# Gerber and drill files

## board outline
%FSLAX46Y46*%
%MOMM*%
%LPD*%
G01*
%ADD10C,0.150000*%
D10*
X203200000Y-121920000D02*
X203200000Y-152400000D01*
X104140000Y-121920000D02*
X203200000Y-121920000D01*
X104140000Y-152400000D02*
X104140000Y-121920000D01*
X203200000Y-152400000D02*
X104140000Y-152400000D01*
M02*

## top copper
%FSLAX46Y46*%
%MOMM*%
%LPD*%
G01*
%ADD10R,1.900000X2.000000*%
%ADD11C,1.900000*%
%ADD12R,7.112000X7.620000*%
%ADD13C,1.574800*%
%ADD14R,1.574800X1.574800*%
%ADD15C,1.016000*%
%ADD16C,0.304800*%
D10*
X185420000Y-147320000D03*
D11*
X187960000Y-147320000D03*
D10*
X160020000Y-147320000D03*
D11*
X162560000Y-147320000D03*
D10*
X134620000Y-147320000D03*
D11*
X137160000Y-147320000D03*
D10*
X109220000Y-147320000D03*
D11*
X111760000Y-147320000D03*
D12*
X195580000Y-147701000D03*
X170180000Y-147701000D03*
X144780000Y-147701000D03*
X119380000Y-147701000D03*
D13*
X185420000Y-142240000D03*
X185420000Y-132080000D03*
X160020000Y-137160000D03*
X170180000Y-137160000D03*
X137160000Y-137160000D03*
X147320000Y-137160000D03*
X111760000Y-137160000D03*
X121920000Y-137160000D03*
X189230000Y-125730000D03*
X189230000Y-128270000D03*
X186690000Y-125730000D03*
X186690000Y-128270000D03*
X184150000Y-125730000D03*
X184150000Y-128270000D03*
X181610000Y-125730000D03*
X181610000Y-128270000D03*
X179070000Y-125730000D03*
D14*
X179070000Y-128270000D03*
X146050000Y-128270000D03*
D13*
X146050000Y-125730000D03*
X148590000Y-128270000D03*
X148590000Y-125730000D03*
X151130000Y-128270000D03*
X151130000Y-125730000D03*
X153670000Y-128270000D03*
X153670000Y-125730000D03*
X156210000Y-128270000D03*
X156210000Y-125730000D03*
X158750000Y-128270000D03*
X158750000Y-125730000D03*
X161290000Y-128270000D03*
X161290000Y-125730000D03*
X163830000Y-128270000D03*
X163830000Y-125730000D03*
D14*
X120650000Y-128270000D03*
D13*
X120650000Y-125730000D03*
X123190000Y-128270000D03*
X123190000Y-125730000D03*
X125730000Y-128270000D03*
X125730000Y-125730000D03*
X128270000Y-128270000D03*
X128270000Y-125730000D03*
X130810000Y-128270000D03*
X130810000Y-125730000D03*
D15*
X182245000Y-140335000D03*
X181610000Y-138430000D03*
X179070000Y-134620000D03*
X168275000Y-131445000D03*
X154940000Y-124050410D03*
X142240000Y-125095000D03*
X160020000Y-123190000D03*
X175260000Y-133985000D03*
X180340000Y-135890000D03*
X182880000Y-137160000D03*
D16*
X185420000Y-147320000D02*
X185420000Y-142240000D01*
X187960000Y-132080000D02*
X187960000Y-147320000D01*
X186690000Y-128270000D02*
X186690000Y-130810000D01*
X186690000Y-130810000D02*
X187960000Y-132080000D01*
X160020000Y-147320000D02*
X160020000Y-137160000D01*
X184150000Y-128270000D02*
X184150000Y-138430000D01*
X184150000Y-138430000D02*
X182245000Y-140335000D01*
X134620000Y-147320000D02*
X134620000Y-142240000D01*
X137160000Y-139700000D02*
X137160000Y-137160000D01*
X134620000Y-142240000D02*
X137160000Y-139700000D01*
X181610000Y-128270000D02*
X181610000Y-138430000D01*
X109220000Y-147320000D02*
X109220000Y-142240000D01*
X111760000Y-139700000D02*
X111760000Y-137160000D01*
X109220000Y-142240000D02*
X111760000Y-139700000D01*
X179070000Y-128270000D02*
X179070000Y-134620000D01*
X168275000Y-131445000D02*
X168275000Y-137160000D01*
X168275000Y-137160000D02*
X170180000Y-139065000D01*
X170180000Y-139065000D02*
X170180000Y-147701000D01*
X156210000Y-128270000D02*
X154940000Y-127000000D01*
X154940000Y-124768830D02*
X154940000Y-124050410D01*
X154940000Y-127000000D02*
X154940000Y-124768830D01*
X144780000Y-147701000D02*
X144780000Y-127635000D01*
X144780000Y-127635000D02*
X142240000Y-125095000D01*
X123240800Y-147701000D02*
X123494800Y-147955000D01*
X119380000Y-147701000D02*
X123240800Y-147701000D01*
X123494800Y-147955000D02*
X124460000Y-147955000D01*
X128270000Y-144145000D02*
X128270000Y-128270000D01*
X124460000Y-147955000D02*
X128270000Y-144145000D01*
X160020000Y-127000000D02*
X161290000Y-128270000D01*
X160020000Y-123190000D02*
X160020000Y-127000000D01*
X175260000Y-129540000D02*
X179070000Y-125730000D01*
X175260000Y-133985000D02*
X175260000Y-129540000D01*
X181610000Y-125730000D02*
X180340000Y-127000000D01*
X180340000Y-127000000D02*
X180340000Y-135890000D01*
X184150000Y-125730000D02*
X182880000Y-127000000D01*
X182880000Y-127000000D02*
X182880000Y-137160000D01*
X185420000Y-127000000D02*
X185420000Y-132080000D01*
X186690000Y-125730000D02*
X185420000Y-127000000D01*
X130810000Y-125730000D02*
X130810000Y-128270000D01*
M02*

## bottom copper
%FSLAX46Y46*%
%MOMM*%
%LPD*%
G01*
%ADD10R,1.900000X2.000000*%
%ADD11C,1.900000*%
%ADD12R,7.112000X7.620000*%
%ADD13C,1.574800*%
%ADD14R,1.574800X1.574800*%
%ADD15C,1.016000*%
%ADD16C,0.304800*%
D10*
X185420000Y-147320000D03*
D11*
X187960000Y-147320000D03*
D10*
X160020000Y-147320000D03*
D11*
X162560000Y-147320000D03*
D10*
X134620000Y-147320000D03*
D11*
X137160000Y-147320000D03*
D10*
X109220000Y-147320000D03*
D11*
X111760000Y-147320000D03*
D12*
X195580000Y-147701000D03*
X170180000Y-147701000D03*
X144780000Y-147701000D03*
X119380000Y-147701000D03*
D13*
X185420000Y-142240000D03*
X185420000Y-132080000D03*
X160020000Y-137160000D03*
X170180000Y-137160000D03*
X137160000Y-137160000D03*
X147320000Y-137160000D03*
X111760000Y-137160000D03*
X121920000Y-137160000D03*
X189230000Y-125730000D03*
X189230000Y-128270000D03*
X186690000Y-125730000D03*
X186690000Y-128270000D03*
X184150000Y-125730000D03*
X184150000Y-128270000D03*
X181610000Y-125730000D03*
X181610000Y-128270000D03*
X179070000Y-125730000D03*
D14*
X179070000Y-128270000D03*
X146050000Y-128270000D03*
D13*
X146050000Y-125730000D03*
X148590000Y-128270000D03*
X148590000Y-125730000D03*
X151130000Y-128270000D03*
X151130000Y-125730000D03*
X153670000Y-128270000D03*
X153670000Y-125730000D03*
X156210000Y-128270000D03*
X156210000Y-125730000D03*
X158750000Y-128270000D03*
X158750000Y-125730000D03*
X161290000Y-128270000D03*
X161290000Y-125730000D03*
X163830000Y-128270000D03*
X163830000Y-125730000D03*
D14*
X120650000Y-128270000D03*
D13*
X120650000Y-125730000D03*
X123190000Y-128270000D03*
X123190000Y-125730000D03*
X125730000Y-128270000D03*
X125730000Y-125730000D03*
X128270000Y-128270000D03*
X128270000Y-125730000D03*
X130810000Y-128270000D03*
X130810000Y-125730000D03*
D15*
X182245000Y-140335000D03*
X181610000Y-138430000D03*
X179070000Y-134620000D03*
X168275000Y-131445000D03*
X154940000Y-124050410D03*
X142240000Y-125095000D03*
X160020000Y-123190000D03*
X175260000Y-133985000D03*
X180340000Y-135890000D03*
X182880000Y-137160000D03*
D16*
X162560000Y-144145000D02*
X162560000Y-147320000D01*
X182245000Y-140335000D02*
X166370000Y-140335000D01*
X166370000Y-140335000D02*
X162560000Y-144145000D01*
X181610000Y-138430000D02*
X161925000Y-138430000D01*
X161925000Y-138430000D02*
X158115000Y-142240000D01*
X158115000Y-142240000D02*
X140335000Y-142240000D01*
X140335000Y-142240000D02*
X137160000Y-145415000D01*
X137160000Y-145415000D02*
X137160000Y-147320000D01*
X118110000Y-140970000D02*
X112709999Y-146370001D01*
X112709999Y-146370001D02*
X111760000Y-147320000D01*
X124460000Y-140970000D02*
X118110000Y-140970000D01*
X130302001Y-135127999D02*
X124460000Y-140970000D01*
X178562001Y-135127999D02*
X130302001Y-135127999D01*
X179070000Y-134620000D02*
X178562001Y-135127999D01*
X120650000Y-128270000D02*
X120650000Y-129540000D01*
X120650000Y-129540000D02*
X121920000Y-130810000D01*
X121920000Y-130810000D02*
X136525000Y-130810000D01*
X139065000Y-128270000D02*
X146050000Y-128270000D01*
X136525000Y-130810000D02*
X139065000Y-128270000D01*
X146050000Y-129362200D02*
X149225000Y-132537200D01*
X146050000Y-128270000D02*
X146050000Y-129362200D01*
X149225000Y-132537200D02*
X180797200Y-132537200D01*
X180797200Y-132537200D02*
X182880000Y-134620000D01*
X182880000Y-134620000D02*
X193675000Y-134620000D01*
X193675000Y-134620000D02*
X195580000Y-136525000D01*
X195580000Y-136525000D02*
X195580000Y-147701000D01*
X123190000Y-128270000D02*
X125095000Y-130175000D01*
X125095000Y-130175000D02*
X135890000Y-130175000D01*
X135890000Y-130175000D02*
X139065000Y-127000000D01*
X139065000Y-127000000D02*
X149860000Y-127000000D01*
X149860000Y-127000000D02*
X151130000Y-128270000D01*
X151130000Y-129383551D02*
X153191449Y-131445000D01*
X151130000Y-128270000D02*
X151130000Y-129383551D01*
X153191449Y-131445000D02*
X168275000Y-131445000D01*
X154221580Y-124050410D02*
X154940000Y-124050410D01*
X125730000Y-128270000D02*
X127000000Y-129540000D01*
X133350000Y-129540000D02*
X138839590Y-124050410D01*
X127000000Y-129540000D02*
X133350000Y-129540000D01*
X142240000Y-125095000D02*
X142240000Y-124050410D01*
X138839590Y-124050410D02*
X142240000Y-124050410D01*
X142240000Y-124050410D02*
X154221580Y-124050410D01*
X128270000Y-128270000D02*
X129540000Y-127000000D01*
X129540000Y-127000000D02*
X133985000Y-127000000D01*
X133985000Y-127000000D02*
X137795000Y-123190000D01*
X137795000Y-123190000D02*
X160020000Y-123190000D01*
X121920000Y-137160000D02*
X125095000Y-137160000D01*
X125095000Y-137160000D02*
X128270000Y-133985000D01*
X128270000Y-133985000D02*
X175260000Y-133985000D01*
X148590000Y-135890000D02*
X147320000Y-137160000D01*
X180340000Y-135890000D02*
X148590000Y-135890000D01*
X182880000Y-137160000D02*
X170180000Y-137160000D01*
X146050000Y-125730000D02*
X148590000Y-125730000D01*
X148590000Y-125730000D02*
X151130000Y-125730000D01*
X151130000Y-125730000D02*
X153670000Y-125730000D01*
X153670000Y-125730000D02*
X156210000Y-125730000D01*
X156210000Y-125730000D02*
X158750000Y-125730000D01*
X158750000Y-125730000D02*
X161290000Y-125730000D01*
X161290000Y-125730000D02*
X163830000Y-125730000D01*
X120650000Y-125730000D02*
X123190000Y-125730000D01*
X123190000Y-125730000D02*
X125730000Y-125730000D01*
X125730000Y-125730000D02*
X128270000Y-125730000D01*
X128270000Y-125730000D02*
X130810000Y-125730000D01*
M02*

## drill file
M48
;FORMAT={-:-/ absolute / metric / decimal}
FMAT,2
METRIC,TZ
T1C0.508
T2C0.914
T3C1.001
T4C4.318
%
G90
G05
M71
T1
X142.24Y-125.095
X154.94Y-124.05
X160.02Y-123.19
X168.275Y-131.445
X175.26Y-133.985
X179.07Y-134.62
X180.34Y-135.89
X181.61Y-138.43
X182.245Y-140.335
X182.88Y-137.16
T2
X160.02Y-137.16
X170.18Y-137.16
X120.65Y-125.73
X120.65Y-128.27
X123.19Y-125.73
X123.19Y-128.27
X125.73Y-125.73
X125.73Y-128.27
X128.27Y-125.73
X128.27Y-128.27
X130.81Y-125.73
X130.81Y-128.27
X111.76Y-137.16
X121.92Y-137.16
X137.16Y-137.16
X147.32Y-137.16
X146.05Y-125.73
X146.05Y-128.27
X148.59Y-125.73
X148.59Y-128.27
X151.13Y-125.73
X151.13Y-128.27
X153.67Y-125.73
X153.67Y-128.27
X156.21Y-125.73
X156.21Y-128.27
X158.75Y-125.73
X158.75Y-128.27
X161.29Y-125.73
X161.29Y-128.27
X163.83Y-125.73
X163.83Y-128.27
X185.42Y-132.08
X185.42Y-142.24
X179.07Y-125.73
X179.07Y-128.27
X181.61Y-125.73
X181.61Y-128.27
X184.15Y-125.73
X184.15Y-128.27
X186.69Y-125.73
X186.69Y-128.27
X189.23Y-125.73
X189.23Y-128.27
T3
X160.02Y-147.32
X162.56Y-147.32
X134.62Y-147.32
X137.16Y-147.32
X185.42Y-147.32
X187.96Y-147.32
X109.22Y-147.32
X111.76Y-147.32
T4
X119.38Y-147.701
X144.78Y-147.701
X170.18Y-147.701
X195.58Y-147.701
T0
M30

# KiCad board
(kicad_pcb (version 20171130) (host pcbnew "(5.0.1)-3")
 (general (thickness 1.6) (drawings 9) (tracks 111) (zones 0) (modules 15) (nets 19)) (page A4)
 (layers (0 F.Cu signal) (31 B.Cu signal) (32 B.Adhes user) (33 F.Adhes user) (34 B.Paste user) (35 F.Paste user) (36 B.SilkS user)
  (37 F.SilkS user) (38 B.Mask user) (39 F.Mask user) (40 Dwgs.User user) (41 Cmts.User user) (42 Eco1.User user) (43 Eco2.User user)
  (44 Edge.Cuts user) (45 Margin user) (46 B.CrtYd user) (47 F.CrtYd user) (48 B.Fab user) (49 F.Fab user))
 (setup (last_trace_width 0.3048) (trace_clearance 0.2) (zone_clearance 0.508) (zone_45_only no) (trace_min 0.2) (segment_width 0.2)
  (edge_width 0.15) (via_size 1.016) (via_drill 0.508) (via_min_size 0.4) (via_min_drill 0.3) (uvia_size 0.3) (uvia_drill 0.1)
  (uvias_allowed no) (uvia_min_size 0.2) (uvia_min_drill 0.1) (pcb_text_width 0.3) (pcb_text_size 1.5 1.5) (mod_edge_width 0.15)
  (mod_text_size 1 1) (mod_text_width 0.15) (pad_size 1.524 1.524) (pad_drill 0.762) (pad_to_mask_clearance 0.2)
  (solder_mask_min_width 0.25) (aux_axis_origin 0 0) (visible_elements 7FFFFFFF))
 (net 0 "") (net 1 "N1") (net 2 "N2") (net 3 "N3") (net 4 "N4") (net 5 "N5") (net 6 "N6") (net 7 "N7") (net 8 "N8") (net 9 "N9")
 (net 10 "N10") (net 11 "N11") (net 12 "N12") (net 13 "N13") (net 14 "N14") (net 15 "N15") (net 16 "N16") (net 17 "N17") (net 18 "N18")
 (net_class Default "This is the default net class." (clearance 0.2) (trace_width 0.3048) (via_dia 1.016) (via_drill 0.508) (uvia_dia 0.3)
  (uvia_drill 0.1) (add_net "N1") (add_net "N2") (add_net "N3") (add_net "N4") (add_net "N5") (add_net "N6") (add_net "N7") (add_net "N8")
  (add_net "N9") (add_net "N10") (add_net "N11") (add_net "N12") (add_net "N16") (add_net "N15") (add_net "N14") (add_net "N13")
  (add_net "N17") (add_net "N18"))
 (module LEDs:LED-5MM (layer F.Cu) (at 185.42 147.32)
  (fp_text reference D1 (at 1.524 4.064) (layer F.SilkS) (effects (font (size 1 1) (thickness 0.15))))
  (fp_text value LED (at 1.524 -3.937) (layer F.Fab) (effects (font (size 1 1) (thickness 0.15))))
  (pad 1 thru_hole rect (at 0 0 90) (size 2 1.9) (drill 1.00076) (layers *.Cu *.Mask F.SilkS) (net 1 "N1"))
  (pad 2 thru_hole circle (at 2.54 0) (size 1.9 1.9) (drill 1.00076) (layers *.Cu *.Mask F.SilkS) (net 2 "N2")))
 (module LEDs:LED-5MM (layer F.Cu) (at 160.02 147.32)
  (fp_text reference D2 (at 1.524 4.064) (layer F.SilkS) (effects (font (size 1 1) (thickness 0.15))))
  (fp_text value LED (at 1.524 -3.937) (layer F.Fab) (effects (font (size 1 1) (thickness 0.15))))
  (pad 1 thru_hole rect (at 0 0 90) (size 2 1.9) (drill 1.00076) (layers *.Cu *.Mask F.SilkS) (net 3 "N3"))
  (pad 2 thru_hole circle (at 2.54 0) (size 1.9 1.9) (drill 1.00076) (layers *.Cu *.Mask F.SilkS) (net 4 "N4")))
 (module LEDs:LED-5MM (layer F.Cu) (at 134.62 147.32)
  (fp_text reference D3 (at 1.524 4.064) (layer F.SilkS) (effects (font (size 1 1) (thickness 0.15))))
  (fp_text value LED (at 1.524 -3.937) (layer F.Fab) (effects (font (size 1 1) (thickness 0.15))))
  (pad 1 thru_hole rect (at 0 0 90) (size 2 1.9) (drill 1.00076) (layers *.Cu *.Mask F.SilkS) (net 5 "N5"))
  (pad 2 thru_hole circle (at 2.54 0) (size 1.9 1.9) (drill 1.00076) (layers *.Cu *.Mask F.SilkS) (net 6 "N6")))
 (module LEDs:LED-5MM (layer F.Cu) (at 109.22 147.32)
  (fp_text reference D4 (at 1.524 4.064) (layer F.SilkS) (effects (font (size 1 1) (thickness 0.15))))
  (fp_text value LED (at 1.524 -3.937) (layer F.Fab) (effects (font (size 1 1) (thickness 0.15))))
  (pad 1 thru_hole rect (at 0 0 90) (size 2 1.9) (drill 1.00076) (layers *.Cu *.Mask F.SilkS) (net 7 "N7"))
  (pad 2 thru_hole circle (at 2.54 0) (size 1.9 1.9) (drill 1.00076) (layers *.Cu *.Mask F.SilkS) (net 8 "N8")))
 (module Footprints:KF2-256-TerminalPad (layer F.Cu) (at 195.58 152.4)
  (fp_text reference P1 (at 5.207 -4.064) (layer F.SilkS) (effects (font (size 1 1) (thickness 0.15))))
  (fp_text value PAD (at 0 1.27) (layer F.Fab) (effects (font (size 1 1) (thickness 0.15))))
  (pad 1 thru_hole rect (at 0 -4.699) (size 7.112 7.62) (drill 4.318) (layers *.Cu *.Mask F.SilkS) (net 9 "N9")))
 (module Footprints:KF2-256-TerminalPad (layer F.Cu) (at 170.18 152.4)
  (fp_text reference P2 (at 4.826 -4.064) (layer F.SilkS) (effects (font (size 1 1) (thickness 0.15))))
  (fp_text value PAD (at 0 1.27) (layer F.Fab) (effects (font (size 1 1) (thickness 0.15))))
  (pad 1 thru_hole rect (at 0 -4.699) (size 7.112 7.62) (drill 4.318) (layers *.Cu *.Mask F.SilkS) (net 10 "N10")))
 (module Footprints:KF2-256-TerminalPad (layer F.Cu) (at 144.78 152.4)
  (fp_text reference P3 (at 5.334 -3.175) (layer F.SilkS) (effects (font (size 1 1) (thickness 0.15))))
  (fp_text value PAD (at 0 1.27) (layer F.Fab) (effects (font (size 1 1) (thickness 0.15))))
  (pad 1 thru_hole rect (at 0 -4.699) (size 7.112 7.62) (drill 4.318) (layers *.Cu *.Mask F.SilkS) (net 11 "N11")))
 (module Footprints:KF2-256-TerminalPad (layer F.Cu) (at 119.38 152.4)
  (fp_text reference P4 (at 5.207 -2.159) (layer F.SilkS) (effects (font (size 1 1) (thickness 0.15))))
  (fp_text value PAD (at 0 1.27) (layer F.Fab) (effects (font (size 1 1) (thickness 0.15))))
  (pad 1 thru_hole rect (at 0 -4.699) (size 7.112 7.62) (drill 4.318) (layers *.Cu *.Mask F.SilkS) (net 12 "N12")))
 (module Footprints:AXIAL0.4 (layer F.Cu) (at 185.42 137.16 90)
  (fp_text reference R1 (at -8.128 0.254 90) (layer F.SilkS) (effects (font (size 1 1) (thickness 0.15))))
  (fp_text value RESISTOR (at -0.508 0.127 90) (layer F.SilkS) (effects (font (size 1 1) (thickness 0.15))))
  (pad 1 thru_hole circle (at -5.08 0 90) (size 1.5748 1.5748) (drill 0.9144) (layers *.Cu *.Mask F.SilkS) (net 1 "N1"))
  (pad 2 thru_hole circle (at 5.08 0 90) (size 1.5748 1.5748) (drill 0.9144) (layers *.Cu *.Mask F.SilkS) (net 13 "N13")))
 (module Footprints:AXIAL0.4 (layer F.Cu) (at 165.1 137.16)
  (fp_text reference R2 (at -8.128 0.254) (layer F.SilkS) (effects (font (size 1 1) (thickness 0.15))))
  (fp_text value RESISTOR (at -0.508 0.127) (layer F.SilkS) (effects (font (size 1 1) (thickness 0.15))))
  (pad 1 thru_hole circle (at -5.08 0) (size 1.5748 1.5748) (drill 0.9144) (layers *.Cu *.Mask F.SilkS) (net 3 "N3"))
  (pad 2 thru_hole circle (at 5.08 0) (size 1.5748 1.5748) (drill 0.9144) (layers *.Cu *.Mask F.SilkS) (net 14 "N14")))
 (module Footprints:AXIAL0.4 (layer F.Cu) (at 142.24 137.16)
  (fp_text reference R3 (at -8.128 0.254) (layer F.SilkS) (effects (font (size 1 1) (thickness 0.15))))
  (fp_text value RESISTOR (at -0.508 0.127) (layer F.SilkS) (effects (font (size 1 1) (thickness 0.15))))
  (pad 1 thru_hole circle (at -5.08 0) (size 1.5748 1.5748) (drill 0.9144) (layers *.Cu *.Mask F.SilkS) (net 5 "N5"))
  (pad 2 thru_hole circle (at 5.08 0) (size 1.5748 1.5748) (drill 0.9144) (layers *.Cu *.Mask F.SilkS) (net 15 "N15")))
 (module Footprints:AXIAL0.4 (layer F.Cu) (at 116.84 137.16)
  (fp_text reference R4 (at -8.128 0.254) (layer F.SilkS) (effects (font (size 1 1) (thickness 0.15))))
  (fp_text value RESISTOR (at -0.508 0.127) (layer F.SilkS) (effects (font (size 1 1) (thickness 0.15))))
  (pad 1 thru_hole circle (at -5.08 0) (size 1.5748 1.5748) (drill 0.9144) (layers *.Cu *.Mask F.SilkS) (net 7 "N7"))
  (pad 2 thru_hole circle (at 5.08 0) (size 1.5748 1.5748) (drill 0.9144) (layers *.Cu *.Mask F.SilkS) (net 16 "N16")))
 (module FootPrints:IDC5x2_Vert (layer F.Cu) (at 184.15 127 180)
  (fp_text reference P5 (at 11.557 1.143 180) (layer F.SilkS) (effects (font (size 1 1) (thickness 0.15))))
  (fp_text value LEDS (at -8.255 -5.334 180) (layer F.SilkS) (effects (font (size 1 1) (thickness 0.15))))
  (pad 10 thru_hole circle (at -5.08 1.27 180) (size 1.5748 1.5748) (drill 0.9144) (layers *.Cu *.Mask F.SilkS))
  (pad 9 thru_hole circle (at -5.08 -1.27 180) (size 1.5748 1.5748) (drill 0.9144) (layers *.Cu *.Mask F.SilkS))
  (pad 8 thru_hole circle (at -2.54 1.27 180) (size 1.5748 1.5748) (drill 0.9144) (layers *.Cu *.Mask F.SilkS) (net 13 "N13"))
  (pad 7 thru_hole circle (at -2.54 -1.27 180) (size 1.5748 1.5748) (drill 0.9144) (layers *.Cu *.Mask F.SilkS) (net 2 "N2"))
  (pad 6 thru_hole circle (at 0 1.27 180) (size 1.5748 1.5748) (drill 0.9144) (layers *.Cu *.Mask F.SilkS) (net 14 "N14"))
  (pad 5 thru_hole circle (at 0 -1.27 180) (size 1.5748 1.5748) (drill 0.9144) (layers *.Cu *.Mask F.SilkS) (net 4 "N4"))
  (pad 4 thru_hole circle (at 2.54 1.27 180) (size 1.5748 1.5748) (drill 0.9144) (layers *.Cu *.Mask F.SilkS) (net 15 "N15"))
  (pad 3 thru_hole circle (at 2.54 -1.27 180) (size 1.5748 1.5748) (drill 0.9144) (layers *.Cu *.Mask F.SilkS) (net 6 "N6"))
  (pad 2 thru_hole circle (at 5.08 1.27 180) (size 1.5748 1.5748) (drill 0.9144) (layers *.Cu *.Mask F.SilkS) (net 16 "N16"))
  (pad 1 thru_hole rect (at 5.08 -1.27 180) (size 1.5748 1.5748) (drill 0.9144) (layers *.Cu *.Mask F.SilkS) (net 8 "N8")))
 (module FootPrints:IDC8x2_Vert (layer F.Cu) (at 154.94 127 180)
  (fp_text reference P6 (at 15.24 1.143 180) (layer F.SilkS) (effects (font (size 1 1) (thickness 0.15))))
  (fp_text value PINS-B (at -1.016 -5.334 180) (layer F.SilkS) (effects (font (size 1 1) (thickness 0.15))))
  (pad 1 thru_hole rect (at 8.89 -1.27 180) (size 1.5748 1.5748) (drill 0.9144) (layers *.Cu *.Mask F.SilkS) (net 9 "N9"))
  (pad 2 thru_hole circle (at 8.89 1.27 180) (size 1.5748 1.5748) (drill 0.9144) (layers *.Cu *.Mask F.SilkS) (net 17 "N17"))
  (pad 3 thru_hole circle (at 6.35 -1.27 180) (size 1.5748 1.5748) (drill 0.9144) (layers *.Cu *.Mask F.SilkS))
  (pad 4 thru_hole circle (at 6.35 1.27 180) (size 1.5748 1.5748) (drill 0.9144) (layers *.Cu *.Mask F.SilkS) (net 17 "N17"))
  (pad 5 thru_hole circle (at 3.81 -1.27 180) (size 1.5748 1.5748) (drill 0.9144) (layers *.Cu *.Mask F.SilkS) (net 10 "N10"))
  (pad 6 thru_hole circle (at 3.81 1.27 180) (size 1.5748 1.5748) (drill 0.9144) (layers *.Cu *.Mask F.SilkS) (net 17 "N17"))
  (pad 7 thru_hole circle (at 1.27 -1.27 180) (size 1.5748 1.5748) (drill 0.9144) (layers *.Cu *.Mask F.SilkS))
  (pad 8 thru_hole circle (at 1.27 1.27 180) (size 1.5748 1.5748) (drill 0.9144) (layers *.Cu *.Mask F.SilkS) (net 17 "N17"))
  (pad 9 thru_hole circle (at -1.27 -1.27 180) (size 1.5748 1.5748) (drill 0.9144) (layers *.Cu *.Mask F.SilkS) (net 11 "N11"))
  (pad 10 thru_hole circle (at -1.27 1.27 180) (size 1.5748 1.5748) (drill 0.9144) (layers *.Cu *.Mask F.SilkS) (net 17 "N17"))
  (pad 11 thru_hole circle (at -3.81 -1.27 180) (size 1.5748 1.5748) (drill 0.9144) (layers *.Cu *.Mask F.SilkS))
  (pad 12 thru_hole circle (at -3.81 1.27 180) (size 1.5748 1.5748) (drill 0.9144) (layers *.Cu *.Mask F.SilkS) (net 17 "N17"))
  (pad 13 thru_hole circle (at -6.35 -1.27 180) (size 1.5748 1.5748) (drill 0.9144) (layers *.Cu *.Mask F.SilkS) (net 12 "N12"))
  (pad 14 thru_hole circle (at -6.35 1.27 180) (size 1.5748 1.5748) (drill 0.9144) (layers *.Cu *.Mask F.SilkS) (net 17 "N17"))
  (pad 15 thru_hole circle (at -8.89 -1.27 180) (size 1.5748 1.5748) (drill 0.9144) (layers *.Cu *.Mask F.SilkS))
  (pad 16 thru_hole circle (at -8.89 1.27 180) (size 1.5748 1.5748) (drill 0.9144) (layers *.Cu *.Mask F.SilkS) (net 17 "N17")))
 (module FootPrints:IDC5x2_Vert (layer F.Cu) (at 125.73 127 180)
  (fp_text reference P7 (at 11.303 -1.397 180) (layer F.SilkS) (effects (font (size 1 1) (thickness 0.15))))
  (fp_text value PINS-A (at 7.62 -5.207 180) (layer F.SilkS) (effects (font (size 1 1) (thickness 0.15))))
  (pad 1 thru_hole rect (at 5.08 -1.27 180) (size 1.5748 1.5748) (drill 0.9144) (layers *.Cu *.Mask F.SilkS) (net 9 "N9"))
  (pad 2 thru_hole circle (at 5.08 1.27 180) (size 1.5748 1.5748) (drill 0.9144) (layers *.Cu *.Mask F.SilkS) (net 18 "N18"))
  (pad 3 thru_hole circle (at 2.54 -1.27 180) (size 1.5748 1.5748) (drill 0.9144) (layers *.Cu *.Mask F.SilkS) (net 10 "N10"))
  (pad 4 thru_hole circle (at 2.54 1.27 180) (size 1.5748 1.5748) (drill 0.9144) (layers *.Cu *.Mask F.SilkS) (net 18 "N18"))
  (pad 5 thru_hole circle (at 0 -1.27 180) (size 1.5748 1.5748) (drill 0.9144) (layers *.Cu *.Mask F.SilkS) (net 11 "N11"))
  (pad 6 thru_hole circle (at 0 1.27 180) (size 1.5748 1.5748) (drill 0.9144) (layers *.Cu *.Mask F.SilkS) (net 18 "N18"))
  (pad 7 thru_hole circle (at -2.54 -1.27 180) (size 1.5748 1.5748) (drill 0.9144) (layers *.Cu *.Mask F.SilkS) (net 12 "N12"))
  (pad 8 thru_hole circle (at -2.54 1.27 180) (size 1.5748 1.5748) (drill 0.9144) (layers *.Cu *.Mask F.SilkS) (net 18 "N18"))
  (pad 9 thru_hole circle (at -5.08 -1.27 180) (size 1.5748 1.5748) (drill 0.9144) (layers *.Cu *.Mask F.SilkS) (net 18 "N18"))
  (pad 10 thru_hole circle (at -5.08 1.27 180) (size 1.5748 1.5748) (drill 0.9144) (layers *.Cu *.Mask F.SilkS) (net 18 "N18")))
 (gr_line (start 203.2 121.92) (end 203.2 152.4) (angle 90) (layer Edge.Cuts) (width 0.15))
 (gr_line (start 104.14 121.92) (end 203.2 121.92) (angle 90) (layer Edge.Cuts) (width 0.15))
 (gr_line (start 104.14 152.4) (end 104.14 121.92) (angle 90) (layer Edge.Cuts) (width 0.15))
 (gr_line (start 203.2 152.4) (end 104.14 152.4) (angle 90) (layer Edge.Cuts) (width 0.15))
 (segment (start 185.42 147.32) (end 185.42 142.24) (width 0.3048) (layer F.Cu) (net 1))
 (segment (start 187.96 132.08) (end 187.96 147.32) (width 0.3048) (layer F.Cu) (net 2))
 (segment (start 186.69 128.27) (end 186.69 130.81) (width 0.3048) (layer F.Cu) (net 2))
 (segment (start 186.69 130.81) (end 187.96 132.08) (width 0.3048) (layer F.Cu) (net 2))
 (segment (start 160.02 147.32) (end 160.02 137.16) (width 0.3048) (layer F.Cu) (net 3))
 (via (at 182.245 140.335) (size 1.016) (drill 0.508) (layers F.Cu B.Cu) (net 4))
 (segment (start 184.15 128.27) (end 184.15 138.43) (width 0.3048) (layer F.Cu) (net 4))
 (segment (start 184.15 138.43) (end 182.245 140.335) (width 0.3048) (layer F.Cu) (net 4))
 (segment (start 162.56 144.145) (end 162.56 147.32) (width 0.3048) (layer B.Cu) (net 4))
 (segment (start 182.245 140.335) (end 166.37 140.335) (width 0.3048) (layer B.Cu) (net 4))
 (segment (start 166.37 140.335) (end 162.56 144.145) (width 0.3048) (layer B.Cu) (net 4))
 (segment (start 134.62 147.32) (end 134.62 142.24) (width 0.3048) (layer F.Cu) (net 5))
 (segment (start 137.16 139.7) (end 137.16 137.16) (width 0.3048) (layer F.Cu) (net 5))
 (segment (start 134.62 142.24) (end 137.16 139.7) (width 0.3048) (layer F.Cu) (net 5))
 (via (at 181.61 138.43) (size 1.016) (drill 0.508) (layers F.Cu B.Cu) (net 6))
 (segment (start 181.61 128.27) (end 181.61 138.43) (width 0.3048) (layer F.Cu) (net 6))
 (segment (start 181.61 138.43) (end 161.925 138.43) (width 0.3048) (layer B.Cu) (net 6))
 (segment (start 161.925 138.43) (end 158.115 142.24) (width 0.3048) (layer B.Cu) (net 6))
 (segment (start 158.115 142.24) (end 140.335 142.24) (width 0.3048) (layer B.Cu) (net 6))
 (segment (start 140.335 142.24) (end 137.16 145.415) (width 0.3048) (layer B.Cu) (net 6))
 (segment (start 137.16 145.415) (end 137.16 147.32) (width 0.3048) (layer B.Cu) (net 6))
 (segment (start 109.22 147.32) (end 109.22 142.24) (width 0.3048) (layer F.Cu) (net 7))
 (segment (start 111.76 139.7) (end 111.76 137.16) (width 0.3048) (layer F.Cu) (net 7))
 (segment (start 109.22 142.24) (end 111.76 139.7) (width 0.3048) (layer F.Cu) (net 7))
 (via (at 179.07 134.62) (size 1.016) (drill 0.508) (layers F.Cu B.Cu) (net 8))
 (segment (start 179.07 128.27) (end 179.07 134.62) (width 0.3048) (layer F.Cu) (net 8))
 (segment (start 118.11 140.97) (end 112.709999 146.370001) (width 0.3048) (layer B.Cu) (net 8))
 (segment (start 112.709999 146.370001) (end 111.76 147.32) (width 0.3048) (layer B.Cu) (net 8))
 (segment (start 124.46 140.97) (end 118.11 140.97) (width 0.3048) (layer B.Cu) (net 8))
 (segment (start 130.302001 135.127999) (end 124.46 140.97) (width 0.3048) (layer B.Cu) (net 8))
 (segment (start 178.562001 135.127999) (end 130.302001 135.127999) (width 0.3048) (layer B.Cu) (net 8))
 (segment (start 179.07 134.62) (end 178.562001 135.127999) (width 0.3048) (layer B.Cu) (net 8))
 (segment (start 120.65 128.27) (end 120.65 129.54) (width 0.3048) (layer B.Cu) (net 9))
 (segment (start 120.65 129.54) (end 121.92 130.81) (width 0.3048) (layer B.Cu) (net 9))
 (segment (start 121.92 130.81) (end 136.525 130.81) (width 0.3048) (layer B.Cu) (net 9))
 (segment (start 139.065 128.27) (end 146.05 128.27) (width 0.3048) (layer B.Cu) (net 9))
 (segment (start 136.525 130.81) (end 139.065 128.27) (width 0.3048) (layer B.Cu) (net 9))
 (segment (start 146.05 129.3622) (end 149.225 132.5372) (width 0.3048) (layer B.Cu) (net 9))
 (segment (start 146.05 128.27) (end 146.05 129.3622) (width 0.3048) (layer B.Cu) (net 9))
 (segment (start 149.225 132.5372) (end 180.7972 132.5372) (width 0.3048) (layer B.Cu) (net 9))
 (segment (start 180.7972 132.5372) (end 182.88 134.62) (width 0.3048) (layer B.Cu) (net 9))
 (segment (start 182.88 134.62) (end 193.675 134.62) (width 0.3048) (layer B.Cu) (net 9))
 (segment (start 193.675 134.62) (end 195.58 136.525) (width 0.3048) (layer B.Cu) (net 9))
 (segment (start 195.58 136.525) (end 195.58 147.701) (width 0.3048) (layer B.Cu) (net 9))
 (segment (start 123.19 128.27) (end 125.095 130.175) (width 0.3048) (layer B.Cu) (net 10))
 (segment (start 125.095 130.175) (end 135.89 130.175) (width 0.3048) (layer B.Cu) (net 10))
 (segment (start 135.89 130.175) (end 139.065 127) (width 0.3048) (layer B.Cu) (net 10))
 (segment (start 139.065 127) (end 149.86 127) (width 0.3048) (layer B.Cu) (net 10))
 (segment (start 149.86 127) (end 151.13 128.27) (width 0.3048) (layer B.Cu) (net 10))
 (segment (start 151.13 129.383551) (end 153.191449 131.445) (width 0.3048) (layer B.Cu) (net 10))
 (segment (start 151.13 128.27) (end 151.13 129.383551) (width 0.3048) (layer B.Cu) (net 10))
 (via (at 168.275 131.445) (size 1.016) (drill 0.508) (layers F.Cu B.Cu) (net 10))
 (segment (start 153.191449 131.445) (end 168.275 131.445) (width 0.3048) (layer B.Cu) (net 10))
 (segment (start 168.275 131.445) (end 168.275 137.16) (width 0.3048) (layer F.Cu) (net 10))
 (segment (start 168.275 137.16) (end 170.18 139.065) (width 0.3048) (layer F.Cu) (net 10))
 (segment (start 170.18 139.065) (end 170.18 147.701) (width 0.3048) (layer F.Cu) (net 10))
 (via (at 154.94 124.05041) (size 1.016) (drill 0.508) (layers F.Cu B.Cu) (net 11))
 (segment (start 154.22158 124.05041) (end 154.94 124.05041) (width 0.3048) (layer B.Cu) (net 11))
 (segment (start 125.73 128.27) (end 127 129.54) (width 0.3048) (layer B.Cu) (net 11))
 (segment (start 156.21 128.27) (end 154.94 127) (width 0.3048) (layer F.Cu) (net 11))
 (segment (start 154.94 124.76883) (end 154.94 124.05041) (width 0.3048) (layer F.Cu) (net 11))
 (segment (start 133.35 129.54) (end 138.83959 124.05041) (width 0.3048) (layer B.Cu) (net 11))
 (segment (start 154.94 127) (end 154.94 124.76883) (width 0.3048) (layer F.Cu) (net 11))
 (segment (start 127 129.54) (end 133.35 129.54) (width 0.3048) (layer B.Cu) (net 11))
 (via (at 142.24 125.095) (size 1.016) (drill 0.508) (layers F.Cu B.Cu) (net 11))
 (segment (start 144.78 147.701) (end 144.78 127.635) (width 0.3048) (layer F.Cu) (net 11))
 (segment (start 144.78 127.635) (end 142.24 125.095) (width 0.3048) (layer F.Cu) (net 11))
 (segment (start 142.24 125.095) (end 142.24 124.05041) (width 0.3048) (layer B.Cu) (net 11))
 (segment (start 138.83959 124.05041) (end 142.24 124.05041) (width 0.3048) (layer B.Cu) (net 11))
 (segment (start 142.24 124.05041) (end 154.22158 124.05041) (width 0.3048) (layer B.Cu) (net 11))
 (segment (start 123.2408 147.701) (end 123.4948 147.955) (width 0.3048) (layer F.Cu) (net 12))
 (segment (start 119.38 147.701) (end 123.2408 147.701) (width 0.3048) (layer F.Cu) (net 12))
 (segment (start 123.4948 147.955) (end 124.46 147.955) (width 0.3048) (layer F.Cu) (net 12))
 (segment (start 128.27 144.145) (end 128.27 128.27) (width 0.3048) (layer F.Cu) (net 12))
 (segment (start 124.46 147.955) (end 128.27 144.145) (width 0.3048) (layer F.Cu) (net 12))
 (segment (start 128.27 128.27) (end 129.54 127) (width 0.3048) (layer B.Cu) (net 12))
 (segment (start 129.54 127) (end 133.985 127) (width 0.3048) (layer B.Cu) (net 12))
 (segment (start 133.985 127) (end 137.795 123.19) (width 0.3048) (layer B.Cu) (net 12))
 (segment (start 137.795 123.19) (end 160.02 123.19) (width 0.3048) (layer B.Cu) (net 12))
 (via (at 160.02 123.19) (size 1.016) (drill 0.508) (layers F.Cu B.Cu) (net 12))
 (segment (start 160.02 127) (end 161.29 128.27) (width 0.3048) (layer F.Cu) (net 12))
 (segment (start 160.02 123.19) (end 160.02 127) (width 0.3048) (layer F.Cu) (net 12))
 (segment (start 121.92 137.16) (end 125.095 137.16) (width 0.3048) (layer B.Cu) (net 16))
 (segment (start 125.095 137.16) (end 128.27 133.985) (width 0.3048) (layer B.Cu) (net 16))
 (via (at 175.26 133.985) (size 1.016) (drill 0.508) (layers F.Cu B.Cu) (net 16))
 (segment (start 128.27 133.985) (end 175.26 133.985) (width 0.3048) (layer B.Cu) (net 16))
 (segment (start 175.26 129.54) (end 179.07 125.73) (width 0.3048) (layer F.Cu) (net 16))
 (segment (start 175.26 133.985) (end 175.26 129.54) (width 0.3048) (layer F.Cu) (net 16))
 (via (at 180.34 135.89) (size 1.016) (drill 0.508) (layers F.Cu B.Cu) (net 15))
 (segment (start 181.61 125.73) (end 180.34 127) (width 0.3048) (layer F.Cu) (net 15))
 (segment (start 180.34 127) (end 180.34 135.89) (width 0.3048) (layer F.Cu) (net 15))
 (segment (start 148.59 135.89) (end 147.32 137.16) (width 0.3048) (layer B.Cu) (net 15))
 (segment (start 180.34 135.89) (end 148.59 135.89) (width 0.3048) (layer B.Cu) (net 15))
 (segment (start 184.15 125.73) (end 182.88 127) (width 0.3048) (layer F.Cu) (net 14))
 (via (at 182.88 137.16) (size 1.016) (drill 0.508) (layers F.Cu B.Cu) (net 14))
 (segment (start 182.88 127) (end 182.88 137.16) (width 0.3048) (layer F.Cu) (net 14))
 (segment (start 182.88 137.16) (end 170.18 137.16) (width 0.3048) (layer B.Cu) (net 14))
 (segment (start 185.42 127) (end 185.42 132.08) (width 0.3048) (layer F.Cu) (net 13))
 (segment (start 186.69 125.73) (end 185.42 127) (width 0.3048) (layer F.Cu) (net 13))
 (segment (start 146.05 125.73) (end 148.59 125.73) (width 0.3048) (layer B.Cu) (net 17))
 (segment (start 148.59 125.73) (end 151.13 125.73) (width 0.3048) (layer B.Cu) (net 17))
 (segment (start 151.13 125.73) (end 153.67 125.73) (width 0.3048) (layer B.Cu) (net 17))
 (segment (start 153.67 125.73) (end 156.21 125.73) (width 0.3048) (layer B.Cu) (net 17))
 (segment (start 156.21 125.73) (end 158.75 125.73) (width 0.3048) (layer B.Cu) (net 17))
 (segment (start 158.75 125.73) (end 161.29 125.73) (width 0.3048) (layer B.Cu) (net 17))
 (segment (start 161.29 125.73) (end 163.83 125.73) (width 0.3048) (layer B.Cu) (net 17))
 (segment (start 120.65 125.73) (end 123.19 125.73) (width 0.3048) (layer B.Cu) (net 18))
 (segment (start 123.19 125.73) (end 125.73 125.73) (width 0.3048) (layer B.Cu) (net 18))
 (segment (start 125.73 125.73) (end 128.27 125.73) (width 0.3048) (layer B.Cu) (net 18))
 (segment (start 128.27 125.73) (end 130.81 125.73) (width 0.3048) (layer B.Cu) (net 18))
 (segment (start 130.81 125.73) (end 130.81 128.27) (width 0.3048) (layer F.Cu) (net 18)))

